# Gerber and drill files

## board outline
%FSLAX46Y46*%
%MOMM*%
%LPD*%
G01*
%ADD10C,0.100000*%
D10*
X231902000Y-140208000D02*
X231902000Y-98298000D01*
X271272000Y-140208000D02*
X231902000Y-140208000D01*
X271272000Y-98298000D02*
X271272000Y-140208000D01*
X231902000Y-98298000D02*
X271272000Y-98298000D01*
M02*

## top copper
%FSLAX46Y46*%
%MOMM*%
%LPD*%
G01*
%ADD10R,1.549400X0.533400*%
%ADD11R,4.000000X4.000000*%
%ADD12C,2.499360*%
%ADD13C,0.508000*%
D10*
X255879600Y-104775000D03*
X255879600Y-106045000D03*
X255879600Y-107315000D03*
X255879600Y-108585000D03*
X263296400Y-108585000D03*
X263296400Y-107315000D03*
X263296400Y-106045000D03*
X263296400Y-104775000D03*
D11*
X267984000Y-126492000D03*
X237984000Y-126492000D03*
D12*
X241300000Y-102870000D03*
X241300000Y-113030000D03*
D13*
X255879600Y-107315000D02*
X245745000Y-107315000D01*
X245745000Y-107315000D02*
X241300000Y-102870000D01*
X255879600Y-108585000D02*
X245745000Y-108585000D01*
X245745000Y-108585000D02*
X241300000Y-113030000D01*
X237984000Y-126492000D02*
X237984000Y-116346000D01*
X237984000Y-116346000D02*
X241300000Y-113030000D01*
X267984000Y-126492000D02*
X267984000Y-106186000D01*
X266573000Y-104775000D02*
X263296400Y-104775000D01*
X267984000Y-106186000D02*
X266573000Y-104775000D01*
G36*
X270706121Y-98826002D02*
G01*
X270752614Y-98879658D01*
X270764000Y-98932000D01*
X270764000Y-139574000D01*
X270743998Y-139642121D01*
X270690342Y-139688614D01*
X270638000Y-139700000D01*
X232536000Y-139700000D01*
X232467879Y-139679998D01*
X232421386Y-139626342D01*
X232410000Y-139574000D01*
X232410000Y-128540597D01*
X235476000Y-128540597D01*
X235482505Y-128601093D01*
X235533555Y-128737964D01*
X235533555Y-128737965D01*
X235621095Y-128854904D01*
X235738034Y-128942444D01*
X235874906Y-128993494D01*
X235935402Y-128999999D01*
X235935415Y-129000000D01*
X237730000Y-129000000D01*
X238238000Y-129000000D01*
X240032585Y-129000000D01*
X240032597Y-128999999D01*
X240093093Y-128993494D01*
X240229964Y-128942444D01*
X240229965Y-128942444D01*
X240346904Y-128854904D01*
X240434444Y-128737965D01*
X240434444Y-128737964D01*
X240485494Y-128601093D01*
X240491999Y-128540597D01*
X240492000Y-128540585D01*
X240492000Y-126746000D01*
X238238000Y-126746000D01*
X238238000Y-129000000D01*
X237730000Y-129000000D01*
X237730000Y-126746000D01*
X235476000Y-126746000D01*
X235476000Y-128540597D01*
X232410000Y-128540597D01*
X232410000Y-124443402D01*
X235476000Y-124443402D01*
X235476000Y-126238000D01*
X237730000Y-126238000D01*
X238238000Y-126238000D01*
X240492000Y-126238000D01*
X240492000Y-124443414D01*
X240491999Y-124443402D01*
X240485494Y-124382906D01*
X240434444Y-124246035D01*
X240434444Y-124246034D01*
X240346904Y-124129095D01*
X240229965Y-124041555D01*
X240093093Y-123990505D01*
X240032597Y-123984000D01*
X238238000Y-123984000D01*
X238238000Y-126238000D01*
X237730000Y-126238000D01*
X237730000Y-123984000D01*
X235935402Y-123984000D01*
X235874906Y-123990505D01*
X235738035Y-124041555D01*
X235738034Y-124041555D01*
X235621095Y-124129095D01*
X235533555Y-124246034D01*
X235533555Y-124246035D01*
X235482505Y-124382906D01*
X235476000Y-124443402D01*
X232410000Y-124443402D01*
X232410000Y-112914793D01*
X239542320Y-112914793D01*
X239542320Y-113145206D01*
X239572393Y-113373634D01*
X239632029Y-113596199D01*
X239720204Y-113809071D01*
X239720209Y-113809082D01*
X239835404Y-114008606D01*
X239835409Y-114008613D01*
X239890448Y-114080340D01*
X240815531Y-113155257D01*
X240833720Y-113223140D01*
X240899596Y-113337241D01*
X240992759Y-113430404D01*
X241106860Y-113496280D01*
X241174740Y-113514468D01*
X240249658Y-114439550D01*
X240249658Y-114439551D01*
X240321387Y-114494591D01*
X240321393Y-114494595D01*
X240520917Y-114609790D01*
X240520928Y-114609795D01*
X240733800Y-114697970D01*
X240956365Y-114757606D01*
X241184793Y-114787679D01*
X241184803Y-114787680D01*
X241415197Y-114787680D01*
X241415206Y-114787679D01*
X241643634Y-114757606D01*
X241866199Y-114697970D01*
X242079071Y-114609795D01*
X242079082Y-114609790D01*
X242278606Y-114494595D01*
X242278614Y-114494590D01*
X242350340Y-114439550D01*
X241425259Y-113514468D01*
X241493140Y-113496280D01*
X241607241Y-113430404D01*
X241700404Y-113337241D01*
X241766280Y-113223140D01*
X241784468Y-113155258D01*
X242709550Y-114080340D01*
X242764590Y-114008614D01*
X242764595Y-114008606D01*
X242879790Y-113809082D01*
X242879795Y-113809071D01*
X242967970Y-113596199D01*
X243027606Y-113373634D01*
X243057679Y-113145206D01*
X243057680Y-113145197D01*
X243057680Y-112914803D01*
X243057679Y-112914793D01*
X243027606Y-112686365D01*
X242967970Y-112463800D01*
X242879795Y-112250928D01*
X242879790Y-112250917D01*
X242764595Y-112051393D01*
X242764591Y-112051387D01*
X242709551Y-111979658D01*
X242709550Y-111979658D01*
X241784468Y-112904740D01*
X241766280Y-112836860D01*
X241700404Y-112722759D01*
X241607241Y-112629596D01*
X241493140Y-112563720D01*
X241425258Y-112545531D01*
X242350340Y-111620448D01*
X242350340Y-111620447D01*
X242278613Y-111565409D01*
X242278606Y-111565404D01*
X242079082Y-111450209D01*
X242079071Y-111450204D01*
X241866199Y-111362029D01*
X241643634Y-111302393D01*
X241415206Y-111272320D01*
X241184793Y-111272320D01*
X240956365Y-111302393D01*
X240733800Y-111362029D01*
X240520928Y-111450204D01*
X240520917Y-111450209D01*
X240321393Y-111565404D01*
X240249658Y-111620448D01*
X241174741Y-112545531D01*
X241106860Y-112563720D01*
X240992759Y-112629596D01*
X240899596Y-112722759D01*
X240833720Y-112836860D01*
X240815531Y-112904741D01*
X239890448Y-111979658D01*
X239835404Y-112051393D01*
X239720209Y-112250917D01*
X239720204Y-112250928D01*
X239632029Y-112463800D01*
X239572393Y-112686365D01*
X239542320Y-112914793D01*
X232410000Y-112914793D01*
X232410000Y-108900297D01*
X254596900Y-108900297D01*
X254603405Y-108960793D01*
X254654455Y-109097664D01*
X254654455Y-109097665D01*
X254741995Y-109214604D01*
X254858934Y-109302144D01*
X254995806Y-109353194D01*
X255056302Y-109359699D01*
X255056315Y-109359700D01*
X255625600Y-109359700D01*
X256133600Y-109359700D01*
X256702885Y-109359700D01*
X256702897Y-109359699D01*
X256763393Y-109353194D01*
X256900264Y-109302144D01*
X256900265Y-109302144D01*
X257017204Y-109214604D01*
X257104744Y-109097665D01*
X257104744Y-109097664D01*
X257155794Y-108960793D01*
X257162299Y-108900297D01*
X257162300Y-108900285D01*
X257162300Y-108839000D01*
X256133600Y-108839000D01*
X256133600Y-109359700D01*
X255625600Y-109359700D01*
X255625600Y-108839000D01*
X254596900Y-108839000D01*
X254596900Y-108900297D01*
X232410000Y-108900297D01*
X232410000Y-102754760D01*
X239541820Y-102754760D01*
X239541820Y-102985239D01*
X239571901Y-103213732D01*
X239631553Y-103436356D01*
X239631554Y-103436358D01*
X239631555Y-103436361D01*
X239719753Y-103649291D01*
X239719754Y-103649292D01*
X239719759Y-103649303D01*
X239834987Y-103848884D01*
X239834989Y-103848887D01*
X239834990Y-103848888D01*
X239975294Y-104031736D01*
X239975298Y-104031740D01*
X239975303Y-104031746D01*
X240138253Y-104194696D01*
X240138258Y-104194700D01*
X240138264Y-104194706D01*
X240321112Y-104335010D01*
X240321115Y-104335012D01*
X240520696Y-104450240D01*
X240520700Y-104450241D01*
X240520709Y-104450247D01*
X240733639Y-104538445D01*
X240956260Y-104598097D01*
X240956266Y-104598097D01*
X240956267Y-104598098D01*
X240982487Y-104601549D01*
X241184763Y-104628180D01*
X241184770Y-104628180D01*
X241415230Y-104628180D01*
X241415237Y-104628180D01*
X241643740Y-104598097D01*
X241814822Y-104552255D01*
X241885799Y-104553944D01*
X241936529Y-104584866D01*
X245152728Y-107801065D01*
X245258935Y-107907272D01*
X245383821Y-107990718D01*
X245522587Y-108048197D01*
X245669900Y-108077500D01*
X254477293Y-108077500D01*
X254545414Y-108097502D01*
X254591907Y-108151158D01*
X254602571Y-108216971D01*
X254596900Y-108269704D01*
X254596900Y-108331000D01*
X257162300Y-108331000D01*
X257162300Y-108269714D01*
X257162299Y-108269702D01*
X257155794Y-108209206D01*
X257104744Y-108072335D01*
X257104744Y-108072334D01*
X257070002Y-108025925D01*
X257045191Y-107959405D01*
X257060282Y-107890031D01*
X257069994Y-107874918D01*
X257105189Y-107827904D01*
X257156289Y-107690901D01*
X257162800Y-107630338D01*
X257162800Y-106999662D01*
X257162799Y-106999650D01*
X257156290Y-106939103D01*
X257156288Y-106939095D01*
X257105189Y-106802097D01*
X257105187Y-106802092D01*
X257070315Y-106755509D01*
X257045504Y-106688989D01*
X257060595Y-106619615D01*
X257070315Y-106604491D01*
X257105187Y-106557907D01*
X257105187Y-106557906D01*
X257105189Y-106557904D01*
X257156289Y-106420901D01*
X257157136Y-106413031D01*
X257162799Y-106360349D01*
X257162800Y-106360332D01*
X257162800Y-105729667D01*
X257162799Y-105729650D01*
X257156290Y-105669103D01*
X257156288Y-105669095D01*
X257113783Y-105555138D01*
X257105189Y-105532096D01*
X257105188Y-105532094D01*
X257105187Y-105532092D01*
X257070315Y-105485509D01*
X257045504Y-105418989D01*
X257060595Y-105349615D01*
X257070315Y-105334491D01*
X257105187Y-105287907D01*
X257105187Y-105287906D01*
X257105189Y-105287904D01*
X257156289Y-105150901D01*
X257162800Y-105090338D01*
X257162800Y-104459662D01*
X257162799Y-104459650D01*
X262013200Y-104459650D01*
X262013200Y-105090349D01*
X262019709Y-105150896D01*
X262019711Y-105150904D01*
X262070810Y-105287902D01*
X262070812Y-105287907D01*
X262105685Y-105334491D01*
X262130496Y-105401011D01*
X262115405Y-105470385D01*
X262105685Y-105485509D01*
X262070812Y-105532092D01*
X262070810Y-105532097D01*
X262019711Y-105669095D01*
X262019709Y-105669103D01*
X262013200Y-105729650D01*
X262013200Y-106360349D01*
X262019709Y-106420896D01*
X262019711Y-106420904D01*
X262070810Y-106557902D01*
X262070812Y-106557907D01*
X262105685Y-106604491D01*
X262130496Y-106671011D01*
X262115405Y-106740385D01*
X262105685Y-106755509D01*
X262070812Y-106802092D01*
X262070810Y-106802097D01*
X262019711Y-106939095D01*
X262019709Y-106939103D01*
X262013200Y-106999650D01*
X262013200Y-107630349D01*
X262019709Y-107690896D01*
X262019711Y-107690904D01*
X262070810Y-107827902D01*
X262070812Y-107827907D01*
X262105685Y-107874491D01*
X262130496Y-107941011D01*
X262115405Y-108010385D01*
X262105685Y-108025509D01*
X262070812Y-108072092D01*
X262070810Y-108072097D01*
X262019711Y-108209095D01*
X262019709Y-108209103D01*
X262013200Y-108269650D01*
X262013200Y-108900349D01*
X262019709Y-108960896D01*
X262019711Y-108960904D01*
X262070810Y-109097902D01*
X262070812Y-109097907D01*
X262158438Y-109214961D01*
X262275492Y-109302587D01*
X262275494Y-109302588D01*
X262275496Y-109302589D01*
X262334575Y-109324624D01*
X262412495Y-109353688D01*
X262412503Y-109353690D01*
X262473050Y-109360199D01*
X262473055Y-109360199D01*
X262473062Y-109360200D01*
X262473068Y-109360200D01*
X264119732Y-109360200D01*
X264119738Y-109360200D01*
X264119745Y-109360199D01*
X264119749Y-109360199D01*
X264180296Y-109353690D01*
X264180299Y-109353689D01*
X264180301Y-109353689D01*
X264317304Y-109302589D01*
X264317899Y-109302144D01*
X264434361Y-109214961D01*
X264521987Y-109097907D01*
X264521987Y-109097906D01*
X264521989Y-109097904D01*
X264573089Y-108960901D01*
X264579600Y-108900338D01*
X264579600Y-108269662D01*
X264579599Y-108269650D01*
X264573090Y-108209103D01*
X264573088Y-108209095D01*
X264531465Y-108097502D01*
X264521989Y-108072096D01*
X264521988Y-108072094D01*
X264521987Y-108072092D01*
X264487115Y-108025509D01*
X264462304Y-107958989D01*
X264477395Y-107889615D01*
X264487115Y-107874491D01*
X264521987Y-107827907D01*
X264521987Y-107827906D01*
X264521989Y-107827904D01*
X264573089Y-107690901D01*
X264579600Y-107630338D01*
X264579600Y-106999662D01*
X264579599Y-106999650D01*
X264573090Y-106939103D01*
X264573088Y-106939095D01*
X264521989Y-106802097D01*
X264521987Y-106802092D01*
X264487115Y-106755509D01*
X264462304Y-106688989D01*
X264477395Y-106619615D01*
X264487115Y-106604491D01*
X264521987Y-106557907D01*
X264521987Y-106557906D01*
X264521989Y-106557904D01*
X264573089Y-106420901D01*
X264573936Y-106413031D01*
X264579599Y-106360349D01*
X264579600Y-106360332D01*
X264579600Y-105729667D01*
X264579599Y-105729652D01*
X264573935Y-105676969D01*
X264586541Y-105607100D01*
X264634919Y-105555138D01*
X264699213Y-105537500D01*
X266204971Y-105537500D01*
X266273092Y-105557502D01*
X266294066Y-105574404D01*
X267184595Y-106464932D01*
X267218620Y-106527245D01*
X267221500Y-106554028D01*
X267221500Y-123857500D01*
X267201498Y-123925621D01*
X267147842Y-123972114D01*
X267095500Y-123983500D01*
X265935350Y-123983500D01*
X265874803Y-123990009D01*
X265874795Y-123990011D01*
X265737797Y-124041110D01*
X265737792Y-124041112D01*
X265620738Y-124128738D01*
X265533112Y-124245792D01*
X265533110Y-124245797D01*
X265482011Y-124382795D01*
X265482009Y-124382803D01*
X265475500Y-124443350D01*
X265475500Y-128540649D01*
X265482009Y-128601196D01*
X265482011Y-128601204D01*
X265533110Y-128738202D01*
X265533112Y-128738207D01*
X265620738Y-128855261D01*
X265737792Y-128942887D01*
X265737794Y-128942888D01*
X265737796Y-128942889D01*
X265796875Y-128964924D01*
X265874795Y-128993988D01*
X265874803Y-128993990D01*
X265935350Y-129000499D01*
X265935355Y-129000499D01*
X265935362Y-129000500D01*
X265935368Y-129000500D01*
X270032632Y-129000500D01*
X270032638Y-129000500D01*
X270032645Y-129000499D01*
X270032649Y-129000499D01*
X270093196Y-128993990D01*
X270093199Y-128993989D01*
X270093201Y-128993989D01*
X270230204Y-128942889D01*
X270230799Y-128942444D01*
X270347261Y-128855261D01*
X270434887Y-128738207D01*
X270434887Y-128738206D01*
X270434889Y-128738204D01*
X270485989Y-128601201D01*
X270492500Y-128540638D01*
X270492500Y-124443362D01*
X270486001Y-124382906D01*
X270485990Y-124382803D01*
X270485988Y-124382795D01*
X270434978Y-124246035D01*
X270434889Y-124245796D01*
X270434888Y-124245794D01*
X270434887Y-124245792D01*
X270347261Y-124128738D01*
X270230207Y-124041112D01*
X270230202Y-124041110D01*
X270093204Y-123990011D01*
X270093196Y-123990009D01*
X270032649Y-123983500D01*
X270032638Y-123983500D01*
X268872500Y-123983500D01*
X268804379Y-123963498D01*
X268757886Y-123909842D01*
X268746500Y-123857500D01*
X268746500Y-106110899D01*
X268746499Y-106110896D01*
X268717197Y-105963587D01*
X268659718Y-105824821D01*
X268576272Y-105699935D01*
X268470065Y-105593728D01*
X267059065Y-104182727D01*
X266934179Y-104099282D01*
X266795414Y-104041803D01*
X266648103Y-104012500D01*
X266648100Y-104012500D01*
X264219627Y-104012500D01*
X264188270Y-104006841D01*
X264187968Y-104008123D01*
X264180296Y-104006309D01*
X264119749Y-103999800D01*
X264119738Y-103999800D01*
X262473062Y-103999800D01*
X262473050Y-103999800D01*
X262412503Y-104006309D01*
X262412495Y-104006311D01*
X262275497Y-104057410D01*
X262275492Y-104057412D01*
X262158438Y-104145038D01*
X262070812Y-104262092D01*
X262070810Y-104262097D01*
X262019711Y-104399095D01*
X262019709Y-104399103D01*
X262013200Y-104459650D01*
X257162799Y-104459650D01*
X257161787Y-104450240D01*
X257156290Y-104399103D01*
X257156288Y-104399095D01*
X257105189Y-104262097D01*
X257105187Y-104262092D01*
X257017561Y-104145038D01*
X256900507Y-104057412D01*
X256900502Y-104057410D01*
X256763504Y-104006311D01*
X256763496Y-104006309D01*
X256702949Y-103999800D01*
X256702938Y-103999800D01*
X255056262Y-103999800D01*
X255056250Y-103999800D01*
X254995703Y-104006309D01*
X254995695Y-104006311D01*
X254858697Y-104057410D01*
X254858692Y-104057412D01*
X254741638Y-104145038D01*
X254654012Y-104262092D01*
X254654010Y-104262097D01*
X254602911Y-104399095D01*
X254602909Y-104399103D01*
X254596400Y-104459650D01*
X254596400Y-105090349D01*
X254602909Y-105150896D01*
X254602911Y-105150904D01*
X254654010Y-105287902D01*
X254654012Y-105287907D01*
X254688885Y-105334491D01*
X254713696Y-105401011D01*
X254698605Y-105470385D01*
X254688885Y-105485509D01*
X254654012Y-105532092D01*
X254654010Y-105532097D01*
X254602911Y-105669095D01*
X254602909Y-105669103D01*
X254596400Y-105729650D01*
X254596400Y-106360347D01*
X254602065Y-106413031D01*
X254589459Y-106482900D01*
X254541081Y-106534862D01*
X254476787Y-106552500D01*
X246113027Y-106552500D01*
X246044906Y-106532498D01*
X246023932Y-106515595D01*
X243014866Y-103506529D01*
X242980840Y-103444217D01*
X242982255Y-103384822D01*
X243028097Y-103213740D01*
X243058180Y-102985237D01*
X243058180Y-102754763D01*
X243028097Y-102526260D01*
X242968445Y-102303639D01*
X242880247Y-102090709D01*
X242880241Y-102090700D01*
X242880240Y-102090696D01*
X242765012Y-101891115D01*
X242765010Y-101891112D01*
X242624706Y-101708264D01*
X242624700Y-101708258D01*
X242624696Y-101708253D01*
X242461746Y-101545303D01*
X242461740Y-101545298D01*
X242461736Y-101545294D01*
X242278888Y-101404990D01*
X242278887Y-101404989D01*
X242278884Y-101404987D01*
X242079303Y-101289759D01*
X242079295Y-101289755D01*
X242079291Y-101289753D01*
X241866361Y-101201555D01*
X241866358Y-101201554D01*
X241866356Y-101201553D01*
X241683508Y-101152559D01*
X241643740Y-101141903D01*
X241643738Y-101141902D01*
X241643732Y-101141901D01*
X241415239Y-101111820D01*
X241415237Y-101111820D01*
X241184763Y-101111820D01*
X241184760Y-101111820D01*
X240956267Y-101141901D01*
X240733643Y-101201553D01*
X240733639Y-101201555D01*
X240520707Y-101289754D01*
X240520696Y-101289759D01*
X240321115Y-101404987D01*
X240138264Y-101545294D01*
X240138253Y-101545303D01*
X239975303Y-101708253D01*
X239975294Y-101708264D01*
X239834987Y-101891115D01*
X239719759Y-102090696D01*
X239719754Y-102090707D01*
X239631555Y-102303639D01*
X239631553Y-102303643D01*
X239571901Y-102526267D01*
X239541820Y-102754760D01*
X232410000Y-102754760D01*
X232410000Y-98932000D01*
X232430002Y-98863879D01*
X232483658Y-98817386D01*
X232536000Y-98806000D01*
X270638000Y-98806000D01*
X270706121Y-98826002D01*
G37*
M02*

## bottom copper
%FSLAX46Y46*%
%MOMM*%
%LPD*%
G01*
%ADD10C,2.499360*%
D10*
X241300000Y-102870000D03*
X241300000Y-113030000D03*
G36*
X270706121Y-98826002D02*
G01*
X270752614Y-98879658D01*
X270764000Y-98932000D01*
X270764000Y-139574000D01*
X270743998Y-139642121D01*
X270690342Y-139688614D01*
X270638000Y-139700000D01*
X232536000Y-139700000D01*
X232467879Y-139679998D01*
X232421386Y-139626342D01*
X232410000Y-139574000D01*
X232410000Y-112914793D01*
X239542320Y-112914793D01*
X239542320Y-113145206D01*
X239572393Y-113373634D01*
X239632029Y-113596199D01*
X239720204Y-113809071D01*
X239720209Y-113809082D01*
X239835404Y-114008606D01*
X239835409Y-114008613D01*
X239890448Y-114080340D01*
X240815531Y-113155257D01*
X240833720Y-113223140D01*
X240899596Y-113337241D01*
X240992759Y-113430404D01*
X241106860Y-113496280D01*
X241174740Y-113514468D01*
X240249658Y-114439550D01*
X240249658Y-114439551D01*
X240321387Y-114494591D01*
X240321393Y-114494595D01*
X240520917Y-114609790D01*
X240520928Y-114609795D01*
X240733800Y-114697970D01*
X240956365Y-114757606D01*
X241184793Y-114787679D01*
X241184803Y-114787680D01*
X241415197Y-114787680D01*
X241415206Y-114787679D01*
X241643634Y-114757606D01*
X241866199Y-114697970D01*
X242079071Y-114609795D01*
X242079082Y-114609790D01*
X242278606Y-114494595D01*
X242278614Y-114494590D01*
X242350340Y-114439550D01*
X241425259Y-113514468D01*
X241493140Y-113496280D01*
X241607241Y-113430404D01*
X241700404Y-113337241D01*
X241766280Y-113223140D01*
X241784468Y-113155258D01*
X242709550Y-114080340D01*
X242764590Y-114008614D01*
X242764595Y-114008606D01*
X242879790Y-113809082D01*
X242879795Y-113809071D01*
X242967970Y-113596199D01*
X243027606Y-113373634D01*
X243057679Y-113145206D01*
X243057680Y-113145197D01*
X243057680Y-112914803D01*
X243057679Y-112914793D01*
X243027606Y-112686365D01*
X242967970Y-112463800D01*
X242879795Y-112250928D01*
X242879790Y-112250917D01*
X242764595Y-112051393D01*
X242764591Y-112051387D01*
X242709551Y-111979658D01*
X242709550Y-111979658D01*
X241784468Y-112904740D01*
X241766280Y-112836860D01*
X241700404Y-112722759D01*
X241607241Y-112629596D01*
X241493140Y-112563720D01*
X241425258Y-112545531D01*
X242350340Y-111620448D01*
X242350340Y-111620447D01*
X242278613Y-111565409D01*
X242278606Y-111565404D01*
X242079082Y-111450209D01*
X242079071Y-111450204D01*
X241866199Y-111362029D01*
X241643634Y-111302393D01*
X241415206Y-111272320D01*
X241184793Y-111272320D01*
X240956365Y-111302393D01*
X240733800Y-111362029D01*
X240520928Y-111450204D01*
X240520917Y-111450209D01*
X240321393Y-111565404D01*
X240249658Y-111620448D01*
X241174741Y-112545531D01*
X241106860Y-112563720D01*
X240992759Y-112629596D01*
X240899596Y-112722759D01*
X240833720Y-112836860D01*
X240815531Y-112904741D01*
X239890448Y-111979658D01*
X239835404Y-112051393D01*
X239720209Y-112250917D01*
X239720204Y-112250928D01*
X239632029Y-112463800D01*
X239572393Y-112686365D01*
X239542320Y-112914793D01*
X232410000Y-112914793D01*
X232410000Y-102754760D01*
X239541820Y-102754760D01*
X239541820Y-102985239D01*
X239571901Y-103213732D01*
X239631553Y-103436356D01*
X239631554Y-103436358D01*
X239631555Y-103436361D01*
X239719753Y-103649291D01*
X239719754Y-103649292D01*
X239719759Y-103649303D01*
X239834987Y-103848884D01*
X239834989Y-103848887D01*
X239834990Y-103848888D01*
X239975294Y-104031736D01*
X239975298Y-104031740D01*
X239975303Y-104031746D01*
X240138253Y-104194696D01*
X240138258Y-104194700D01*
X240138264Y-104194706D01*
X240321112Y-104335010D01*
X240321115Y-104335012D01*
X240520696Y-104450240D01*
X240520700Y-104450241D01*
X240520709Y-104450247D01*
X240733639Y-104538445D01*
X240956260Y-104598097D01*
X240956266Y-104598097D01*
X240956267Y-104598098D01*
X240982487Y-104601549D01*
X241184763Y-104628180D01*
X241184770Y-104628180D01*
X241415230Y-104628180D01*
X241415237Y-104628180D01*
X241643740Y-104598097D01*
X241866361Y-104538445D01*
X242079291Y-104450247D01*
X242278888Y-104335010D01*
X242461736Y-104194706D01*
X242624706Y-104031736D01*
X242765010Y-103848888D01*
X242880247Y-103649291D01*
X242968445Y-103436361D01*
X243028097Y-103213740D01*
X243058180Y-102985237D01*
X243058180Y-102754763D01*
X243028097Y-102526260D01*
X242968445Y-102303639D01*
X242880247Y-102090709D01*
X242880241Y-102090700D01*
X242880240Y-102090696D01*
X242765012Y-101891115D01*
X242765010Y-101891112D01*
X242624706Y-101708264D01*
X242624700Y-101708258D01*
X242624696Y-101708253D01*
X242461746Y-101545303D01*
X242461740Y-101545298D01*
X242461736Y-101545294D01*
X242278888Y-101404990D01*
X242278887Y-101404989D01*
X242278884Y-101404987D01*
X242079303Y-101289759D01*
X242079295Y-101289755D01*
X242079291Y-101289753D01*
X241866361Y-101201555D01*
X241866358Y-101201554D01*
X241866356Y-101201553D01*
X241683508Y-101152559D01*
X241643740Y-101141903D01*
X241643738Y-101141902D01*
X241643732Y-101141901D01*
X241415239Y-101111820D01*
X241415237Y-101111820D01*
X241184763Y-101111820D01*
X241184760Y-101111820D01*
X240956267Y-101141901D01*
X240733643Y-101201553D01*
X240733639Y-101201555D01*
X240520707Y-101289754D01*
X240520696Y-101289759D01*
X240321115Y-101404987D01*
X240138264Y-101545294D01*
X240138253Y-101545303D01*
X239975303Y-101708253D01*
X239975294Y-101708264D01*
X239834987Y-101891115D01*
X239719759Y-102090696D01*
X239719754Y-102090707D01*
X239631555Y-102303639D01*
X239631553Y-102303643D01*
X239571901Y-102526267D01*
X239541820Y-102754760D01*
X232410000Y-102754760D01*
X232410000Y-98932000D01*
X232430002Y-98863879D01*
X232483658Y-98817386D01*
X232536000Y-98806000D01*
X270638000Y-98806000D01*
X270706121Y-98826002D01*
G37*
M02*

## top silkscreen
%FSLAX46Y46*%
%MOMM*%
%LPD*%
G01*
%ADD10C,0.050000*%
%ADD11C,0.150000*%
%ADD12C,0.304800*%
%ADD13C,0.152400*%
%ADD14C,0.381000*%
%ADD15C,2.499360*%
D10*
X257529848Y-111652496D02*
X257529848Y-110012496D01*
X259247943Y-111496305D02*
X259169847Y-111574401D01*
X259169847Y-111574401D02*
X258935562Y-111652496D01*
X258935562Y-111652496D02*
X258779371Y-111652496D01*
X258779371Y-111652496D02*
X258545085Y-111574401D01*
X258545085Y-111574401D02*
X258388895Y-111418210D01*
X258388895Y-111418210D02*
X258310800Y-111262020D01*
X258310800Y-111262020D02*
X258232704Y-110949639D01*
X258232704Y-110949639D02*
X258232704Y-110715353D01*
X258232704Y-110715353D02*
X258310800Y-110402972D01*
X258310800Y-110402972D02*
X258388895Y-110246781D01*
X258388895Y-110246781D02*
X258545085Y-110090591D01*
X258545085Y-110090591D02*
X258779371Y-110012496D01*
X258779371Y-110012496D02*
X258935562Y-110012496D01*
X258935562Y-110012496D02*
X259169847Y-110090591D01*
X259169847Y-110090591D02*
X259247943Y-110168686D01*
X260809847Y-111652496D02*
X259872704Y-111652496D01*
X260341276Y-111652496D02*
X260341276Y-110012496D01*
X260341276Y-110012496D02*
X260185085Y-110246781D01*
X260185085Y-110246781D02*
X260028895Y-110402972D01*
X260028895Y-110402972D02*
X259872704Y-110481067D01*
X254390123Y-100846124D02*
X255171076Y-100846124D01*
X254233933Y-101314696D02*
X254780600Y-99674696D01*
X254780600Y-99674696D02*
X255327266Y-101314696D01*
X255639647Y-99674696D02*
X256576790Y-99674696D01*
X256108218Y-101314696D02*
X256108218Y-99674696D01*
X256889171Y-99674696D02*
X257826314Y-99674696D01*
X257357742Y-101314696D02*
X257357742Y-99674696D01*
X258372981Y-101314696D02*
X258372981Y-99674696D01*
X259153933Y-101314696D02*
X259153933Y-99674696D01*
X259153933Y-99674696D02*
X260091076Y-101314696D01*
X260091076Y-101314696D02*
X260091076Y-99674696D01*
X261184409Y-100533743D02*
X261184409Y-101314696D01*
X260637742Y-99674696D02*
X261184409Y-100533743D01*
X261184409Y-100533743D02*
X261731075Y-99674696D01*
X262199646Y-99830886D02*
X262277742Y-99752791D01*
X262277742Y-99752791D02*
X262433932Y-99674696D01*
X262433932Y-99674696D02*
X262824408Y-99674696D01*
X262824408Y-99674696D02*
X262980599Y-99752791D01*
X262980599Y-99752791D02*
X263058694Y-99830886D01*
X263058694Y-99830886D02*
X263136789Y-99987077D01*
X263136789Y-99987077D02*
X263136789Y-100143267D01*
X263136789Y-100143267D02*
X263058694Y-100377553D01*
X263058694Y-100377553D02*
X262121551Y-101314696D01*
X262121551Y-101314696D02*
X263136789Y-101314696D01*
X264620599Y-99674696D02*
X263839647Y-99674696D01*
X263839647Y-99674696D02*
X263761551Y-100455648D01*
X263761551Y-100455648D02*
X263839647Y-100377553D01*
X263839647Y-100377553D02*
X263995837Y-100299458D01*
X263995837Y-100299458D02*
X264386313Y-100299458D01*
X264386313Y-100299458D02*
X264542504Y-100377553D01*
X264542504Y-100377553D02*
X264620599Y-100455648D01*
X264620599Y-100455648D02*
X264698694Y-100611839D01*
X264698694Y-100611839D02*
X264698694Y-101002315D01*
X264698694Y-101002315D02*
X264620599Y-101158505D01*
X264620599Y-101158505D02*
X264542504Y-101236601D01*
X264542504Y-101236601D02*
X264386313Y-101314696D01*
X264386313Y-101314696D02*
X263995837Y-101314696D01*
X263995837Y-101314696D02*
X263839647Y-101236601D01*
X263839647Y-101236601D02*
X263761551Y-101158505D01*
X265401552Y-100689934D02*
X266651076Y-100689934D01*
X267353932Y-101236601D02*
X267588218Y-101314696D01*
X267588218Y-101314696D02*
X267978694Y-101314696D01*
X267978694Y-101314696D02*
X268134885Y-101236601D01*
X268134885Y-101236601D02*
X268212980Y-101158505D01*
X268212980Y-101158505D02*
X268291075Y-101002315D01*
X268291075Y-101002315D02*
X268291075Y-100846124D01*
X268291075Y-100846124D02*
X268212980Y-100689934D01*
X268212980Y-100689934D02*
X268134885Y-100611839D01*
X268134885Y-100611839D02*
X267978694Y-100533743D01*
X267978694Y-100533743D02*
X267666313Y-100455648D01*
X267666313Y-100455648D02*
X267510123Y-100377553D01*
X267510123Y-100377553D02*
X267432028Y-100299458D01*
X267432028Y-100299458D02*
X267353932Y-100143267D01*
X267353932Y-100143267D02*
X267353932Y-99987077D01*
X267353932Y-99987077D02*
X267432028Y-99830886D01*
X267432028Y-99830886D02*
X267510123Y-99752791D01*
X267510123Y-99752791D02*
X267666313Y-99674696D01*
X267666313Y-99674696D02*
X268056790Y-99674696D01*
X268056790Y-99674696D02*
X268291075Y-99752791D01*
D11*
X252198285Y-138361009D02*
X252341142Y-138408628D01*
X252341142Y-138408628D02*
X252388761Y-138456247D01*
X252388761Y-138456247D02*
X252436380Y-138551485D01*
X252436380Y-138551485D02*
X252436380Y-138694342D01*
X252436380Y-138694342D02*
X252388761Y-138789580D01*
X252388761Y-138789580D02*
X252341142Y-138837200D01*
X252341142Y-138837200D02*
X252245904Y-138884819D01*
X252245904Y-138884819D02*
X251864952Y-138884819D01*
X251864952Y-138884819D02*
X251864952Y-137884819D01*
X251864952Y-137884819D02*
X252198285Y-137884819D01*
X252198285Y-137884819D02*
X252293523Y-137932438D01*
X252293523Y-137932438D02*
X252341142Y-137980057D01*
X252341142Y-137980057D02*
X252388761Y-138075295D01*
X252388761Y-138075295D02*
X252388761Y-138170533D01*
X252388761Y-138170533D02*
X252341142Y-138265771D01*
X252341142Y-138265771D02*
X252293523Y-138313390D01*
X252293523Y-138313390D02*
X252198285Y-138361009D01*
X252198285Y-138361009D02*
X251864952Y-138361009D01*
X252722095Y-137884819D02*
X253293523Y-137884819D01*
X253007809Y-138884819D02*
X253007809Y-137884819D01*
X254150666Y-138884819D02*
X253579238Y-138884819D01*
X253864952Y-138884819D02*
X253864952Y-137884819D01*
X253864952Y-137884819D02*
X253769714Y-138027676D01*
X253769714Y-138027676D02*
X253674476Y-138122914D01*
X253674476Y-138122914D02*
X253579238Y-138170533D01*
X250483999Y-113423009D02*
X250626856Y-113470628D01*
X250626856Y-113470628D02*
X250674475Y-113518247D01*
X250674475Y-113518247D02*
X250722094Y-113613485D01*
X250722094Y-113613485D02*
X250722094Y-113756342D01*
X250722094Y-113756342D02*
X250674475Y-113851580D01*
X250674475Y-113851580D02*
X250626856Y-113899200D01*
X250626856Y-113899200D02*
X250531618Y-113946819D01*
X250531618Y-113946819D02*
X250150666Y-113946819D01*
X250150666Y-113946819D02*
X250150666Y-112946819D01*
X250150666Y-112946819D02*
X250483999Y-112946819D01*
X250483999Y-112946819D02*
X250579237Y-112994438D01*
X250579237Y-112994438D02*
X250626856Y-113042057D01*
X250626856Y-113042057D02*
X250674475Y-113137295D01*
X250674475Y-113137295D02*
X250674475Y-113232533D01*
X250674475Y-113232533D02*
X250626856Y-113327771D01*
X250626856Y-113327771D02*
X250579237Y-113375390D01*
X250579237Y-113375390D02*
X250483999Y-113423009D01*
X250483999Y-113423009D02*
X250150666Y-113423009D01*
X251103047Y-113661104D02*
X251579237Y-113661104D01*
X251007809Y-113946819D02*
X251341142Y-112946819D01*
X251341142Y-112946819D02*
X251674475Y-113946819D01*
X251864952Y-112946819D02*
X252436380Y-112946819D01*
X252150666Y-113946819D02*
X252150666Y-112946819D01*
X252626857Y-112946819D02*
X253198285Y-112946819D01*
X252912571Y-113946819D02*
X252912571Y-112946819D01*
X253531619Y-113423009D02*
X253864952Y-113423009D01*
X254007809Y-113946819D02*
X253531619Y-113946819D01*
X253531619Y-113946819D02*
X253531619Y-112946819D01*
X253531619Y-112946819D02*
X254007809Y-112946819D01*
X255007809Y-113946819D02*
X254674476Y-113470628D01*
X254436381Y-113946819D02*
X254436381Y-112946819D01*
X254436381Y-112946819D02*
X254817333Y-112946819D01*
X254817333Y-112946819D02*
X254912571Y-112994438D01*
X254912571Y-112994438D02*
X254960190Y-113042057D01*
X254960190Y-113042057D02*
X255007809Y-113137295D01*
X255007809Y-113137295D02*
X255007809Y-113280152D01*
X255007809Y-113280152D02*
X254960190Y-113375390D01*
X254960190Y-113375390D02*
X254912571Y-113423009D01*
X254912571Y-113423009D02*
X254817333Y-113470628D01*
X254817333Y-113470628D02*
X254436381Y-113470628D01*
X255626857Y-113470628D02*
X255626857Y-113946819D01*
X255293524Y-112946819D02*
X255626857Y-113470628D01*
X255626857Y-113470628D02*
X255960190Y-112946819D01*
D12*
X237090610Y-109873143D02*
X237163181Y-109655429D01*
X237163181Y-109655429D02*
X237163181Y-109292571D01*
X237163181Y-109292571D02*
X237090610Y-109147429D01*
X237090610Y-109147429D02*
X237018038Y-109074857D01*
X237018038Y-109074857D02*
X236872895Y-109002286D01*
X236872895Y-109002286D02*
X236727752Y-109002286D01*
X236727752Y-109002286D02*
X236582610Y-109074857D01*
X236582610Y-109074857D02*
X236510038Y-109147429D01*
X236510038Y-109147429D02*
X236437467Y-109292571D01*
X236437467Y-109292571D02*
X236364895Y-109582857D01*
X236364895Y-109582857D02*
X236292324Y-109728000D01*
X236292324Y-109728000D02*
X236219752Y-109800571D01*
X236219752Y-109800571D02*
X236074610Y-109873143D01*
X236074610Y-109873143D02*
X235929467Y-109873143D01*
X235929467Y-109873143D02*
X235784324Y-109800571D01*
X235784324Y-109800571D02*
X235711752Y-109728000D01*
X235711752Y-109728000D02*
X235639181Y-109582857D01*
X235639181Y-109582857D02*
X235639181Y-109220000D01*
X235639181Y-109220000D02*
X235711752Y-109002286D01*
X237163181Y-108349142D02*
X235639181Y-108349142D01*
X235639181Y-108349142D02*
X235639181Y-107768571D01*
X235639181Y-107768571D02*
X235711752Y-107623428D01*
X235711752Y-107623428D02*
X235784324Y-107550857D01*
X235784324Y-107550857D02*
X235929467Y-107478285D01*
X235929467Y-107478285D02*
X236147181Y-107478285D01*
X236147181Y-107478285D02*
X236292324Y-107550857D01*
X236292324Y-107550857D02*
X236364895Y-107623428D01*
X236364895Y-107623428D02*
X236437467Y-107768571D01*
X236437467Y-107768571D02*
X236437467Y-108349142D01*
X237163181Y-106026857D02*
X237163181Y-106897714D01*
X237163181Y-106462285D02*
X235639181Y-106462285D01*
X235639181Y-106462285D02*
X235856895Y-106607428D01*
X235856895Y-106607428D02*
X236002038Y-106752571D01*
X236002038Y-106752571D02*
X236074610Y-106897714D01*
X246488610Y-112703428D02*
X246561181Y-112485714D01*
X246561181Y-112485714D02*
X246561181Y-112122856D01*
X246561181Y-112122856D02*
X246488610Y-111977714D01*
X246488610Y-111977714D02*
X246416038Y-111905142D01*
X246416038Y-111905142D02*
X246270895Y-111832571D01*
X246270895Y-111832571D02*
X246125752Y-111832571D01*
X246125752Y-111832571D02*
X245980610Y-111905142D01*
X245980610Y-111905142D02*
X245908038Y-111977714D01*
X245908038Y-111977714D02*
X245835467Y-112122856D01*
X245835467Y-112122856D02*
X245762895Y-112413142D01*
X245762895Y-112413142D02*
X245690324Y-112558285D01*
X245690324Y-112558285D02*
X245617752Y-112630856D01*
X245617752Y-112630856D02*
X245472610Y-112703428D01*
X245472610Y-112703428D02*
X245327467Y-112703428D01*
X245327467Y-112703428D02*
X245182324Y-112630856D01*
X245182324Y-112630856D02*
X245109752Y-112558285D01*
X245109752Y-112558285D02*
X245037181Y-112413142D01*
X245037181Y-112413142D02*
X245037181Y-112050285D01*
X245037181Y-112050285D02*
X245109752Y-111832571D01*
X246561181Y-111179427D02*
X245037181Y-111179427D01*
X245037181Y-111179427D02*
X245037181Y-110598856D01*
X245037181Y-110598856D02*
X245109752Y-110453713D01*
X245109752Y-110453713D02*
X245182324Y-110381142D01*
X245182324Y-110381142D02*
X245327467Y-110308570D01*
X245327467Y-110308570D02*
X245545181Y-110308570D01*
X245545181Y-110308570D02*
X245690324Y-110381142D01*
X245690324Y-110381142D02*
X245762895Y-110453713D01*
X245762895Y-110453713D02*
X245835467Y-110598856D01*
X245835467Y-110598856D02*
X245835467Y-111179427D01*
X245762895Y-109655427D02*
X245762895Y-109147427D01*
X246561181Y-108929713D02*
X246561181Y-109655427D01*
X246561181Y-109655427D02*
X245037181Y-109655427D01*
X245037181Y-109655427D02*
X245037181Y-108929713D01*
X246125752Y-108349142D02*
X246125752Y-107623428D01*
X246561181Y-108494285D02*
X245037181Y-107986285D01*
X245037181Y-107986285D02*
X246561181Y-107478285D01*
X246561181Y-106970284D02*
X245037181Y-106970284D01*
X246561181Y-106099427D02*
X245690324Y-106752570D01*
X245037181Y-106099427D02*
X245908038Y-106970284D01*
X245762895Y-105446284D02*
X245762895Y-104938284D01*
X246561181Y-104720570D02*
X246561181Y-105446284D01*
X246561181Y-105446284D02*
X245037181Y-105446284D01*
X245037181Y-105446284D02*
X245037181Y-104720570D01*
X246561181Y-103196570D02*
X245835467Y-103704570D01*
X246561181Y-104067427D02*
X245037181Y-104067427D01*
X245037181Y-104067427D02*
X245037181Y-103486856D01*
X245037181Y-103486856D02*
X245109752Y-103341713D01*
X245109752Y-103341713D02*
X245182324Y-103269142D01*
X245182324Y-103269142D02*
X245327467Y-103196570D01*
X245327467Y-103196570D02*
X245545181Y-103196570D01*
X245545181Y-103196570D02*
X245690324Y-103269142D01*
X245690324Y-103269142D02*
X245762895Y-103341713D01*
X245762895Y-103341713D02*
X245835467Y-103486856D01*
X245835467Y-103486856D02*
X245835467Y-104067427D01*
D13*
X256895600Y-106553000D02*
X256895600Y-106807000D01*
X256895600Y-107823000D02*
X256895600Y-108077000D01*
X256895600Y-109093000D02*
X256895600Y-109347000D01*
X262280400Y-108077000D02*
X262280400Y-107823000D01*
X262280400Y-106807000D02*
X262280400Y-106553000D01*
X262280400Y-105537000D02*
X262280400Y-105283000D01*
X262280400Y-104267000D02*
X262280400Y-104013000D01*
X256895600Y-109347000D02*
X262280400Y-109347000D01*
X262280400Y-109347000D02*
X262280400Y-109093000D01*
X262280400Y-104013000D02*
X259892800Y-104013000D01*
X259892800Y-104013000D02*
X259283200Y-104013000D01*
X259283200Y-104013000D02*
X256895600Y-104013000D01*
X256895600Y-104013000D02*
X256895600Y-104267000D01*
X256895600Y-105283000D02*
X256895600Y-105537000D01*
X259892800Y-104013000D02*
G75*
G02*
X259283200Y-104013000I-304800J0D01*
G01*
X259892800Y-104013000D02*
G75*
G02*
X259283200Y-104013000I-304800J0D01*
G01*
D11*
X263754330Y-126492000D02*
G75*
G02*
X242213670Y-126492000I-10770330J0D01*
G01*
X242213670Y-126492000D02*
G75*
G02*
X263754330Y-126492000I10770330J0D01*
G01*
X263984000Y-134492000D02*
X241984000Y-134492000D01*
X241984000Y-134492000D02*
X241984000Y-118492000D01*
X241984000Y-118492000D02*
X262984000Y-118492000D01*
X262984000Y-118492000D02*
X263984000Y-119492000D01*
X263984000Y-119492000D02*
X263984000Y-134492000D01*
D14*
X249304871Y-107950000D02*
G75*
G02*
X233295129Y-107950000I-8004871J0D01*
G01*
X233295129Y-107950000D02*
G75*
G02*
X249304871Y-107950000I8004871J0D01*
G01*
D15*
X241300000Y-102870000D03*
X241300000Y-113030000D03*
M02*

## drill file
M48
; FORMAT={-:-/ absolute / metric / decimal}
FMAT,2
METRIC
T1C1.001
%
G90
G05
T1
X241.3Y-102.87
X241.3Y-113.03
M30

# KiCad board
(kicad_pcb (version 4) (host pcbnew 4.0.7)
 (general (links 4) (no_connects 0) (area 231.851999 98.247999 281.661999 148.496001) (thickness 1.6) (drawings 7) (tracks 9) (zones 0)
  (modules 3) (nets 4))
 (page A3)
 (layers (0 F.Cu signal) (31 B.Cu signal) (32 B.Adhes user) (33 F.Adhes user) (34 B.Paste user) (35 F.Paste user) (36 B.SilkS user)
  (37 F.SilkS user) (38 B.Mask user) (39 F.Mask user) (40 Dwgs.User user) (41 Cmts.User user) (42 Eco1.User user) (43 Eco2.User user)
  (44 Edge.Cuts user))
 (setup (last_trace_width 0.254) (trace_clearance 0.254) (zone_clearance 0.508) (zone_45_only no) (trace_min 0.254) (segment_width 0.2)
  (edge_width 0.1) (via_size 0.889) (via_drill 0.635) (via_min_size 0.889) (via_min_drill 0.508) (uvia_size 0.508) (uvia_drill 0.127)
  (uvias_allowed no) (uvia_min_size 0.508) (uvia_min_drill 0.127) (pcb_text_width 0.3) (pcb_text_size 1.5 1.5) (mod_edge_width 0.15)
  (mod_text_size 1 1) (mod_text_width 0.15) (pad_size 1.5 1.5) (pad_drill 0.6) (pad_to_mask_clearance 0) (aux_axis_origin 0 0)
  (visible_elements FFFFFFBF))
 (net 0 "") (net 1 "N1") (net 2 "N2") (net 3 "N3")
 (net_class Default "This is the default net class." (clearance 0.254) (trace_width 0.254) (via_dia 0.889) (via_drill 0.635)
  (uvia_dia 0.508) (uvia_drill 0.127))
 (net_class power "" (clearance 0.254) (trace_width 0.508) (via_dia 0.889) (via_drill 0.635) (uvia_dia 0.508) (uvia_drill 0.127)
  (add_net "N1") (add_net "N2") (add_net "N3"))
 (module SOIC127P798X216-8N (layer F.Cu) (at 259.588 106.68) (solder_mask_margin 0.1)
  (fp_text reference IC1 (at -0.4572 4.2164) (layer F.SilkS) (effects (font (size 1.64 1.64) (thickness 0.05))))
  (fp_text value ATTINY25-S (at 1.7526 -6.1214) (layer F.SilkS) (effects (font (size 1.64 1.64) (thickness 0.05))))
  (fp_line (start -2.6924 -0.127) (end -2.6924 0.127) (layer F.SilkS) (width 0.1524))
  (fp_line (start -2.6924 1.143) (end -2.6924 1.397) (layer F.SilkS) (width 0.1524))
  (fp_line (start -2.6924 2.413) (end -2.6924 2.667) (layer F.SilkS) (width 0.1524))
  (fp_line (start 2.6924 1.397) (end 2.6924 1.143) (layer F.SilkS) (width 0.1524))
  (fp_line (start 2.6924 0.127) (end 2.6924 -0.127) (layer F.SilkS) (width 0.1524))
  (fp_line (start 2.6924 -1.143) (end 2.6924 -1.397) (layer F.SilkS) (width 0.1524))
  (fp_line (start 2.6924 -2.413) (end 2.6924 -2.667) (layer F.SilkS) (width 0.1524))
  (fp_line (start -2.6924 2.667) (end 2.6924 2.667) (layer F.SilkS) (width 0.1524))
  (fp_line (start 2.6924 2.667) (end 2.6924 2.413) (layer F.SilkS) (width 0.1524))
  (fp_line (start 2.6924 -2.667) (end 0.3048 -2.667) (layer F.SilkS) (width 0.1524))
  (fp_line (start 0.3048 -2.667) (end -0.3048 -2.667) (layer F.SilkS) (width 0.1524))
  (fp_line (start -0.3048 -2.667) (end -2.6924 -2.667) (layer F.SilkS) (width 0.1524))
  (fp_line (start -2.6924 -2.667) (end -2.6924 -2.413) (layer F.SilkS) (width 0.1524))
  (fp_line (start -2.6924 -1.397) (end -2.6924 -1.143) (layer F.SilkS) (width 0.1524))
  (fp_arc (start 0 -2.667) (end -0.3048 -2.667) (angle -180) (layer F.SilkS) (width 0.1524))
  (fp_arc (start 0 -2.667) (end -0.3048 -2.667) (angle -180) (layer F.SilkS) (width 0.1524))
  (pad 1 smd rect (at -3.7084 -1.905) (size 1.5494 0.5334) (layers F.Cu F.Paste F.Mask) (solder_mask_margin 0.2))
  (pad 2 smd rect (at -3.7084 -0.635) (size 1.5494 0.5334) (layers F.Cu F.Paste F.Mask) (solder_mask_margin 0.2))
  (pad 3 smd rect (at -3.7084 0.635) (size 1.5494 0.5334) (layers F.Cu F.Paste F.Mask) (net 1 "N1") (solder_mask_margin 0.2))
  (pad 4 smd rect (at -3.7084 1.905) (size 1.5494 0.5334) (layers F.Cu F.Paste F.Mask) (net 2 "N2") (solder_mask_margin 0.2))
  (pad 5 smd rect (at 3.7084 1.905) (size 1.5494 0.5334) (layers F.Cu F.Paste F.Mask) (solder_mask_margin 0.2))
  (pad 6 smd rect (at 3.7084 0.635) (size 1.5494 0.5334) (layers F.Cu F.Paste F.Mask) (solder_mask_margin 0.2))
  (pad 7 smd rect (at 3.7084 -0.635) (size 1.5494 0.5334) (layers F.Cu F.Paste F.Mask) (solder_mask_margin 0.2))
  (pad 8 smd rect (at 3.7084 -1.905) (size 1.5494 0.5334) (layers F.Cu F.Paste F.Mask) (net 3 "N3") (solder_mask_margin 0.2)))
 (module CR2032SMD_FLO (layer F.Cu) (at 252.984 126.492 180)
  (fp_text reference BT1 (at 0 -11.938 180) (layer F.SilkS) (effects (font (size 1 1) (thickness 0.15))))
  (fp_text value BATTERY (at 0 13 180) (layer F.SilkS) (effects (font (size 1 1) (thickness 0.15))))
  (fp_circle (center 0 0) (end -4 -10) (layer F.SilkS) (width 0.15))
  (fp_line (start -11 -8) (end 11 -8) (layer F.SilkS) (width 0.15))
  (fp_line (start 11 -8) (end 11 8) (layer F.SilkS) (width 0.15))
  (fp_line (start 11 8) (end -10 8) (layer F.SilkS) (width 0.15))
  (fp_line (start -10 8) (end -11 7) (layer F.SilkS) (width 0.15))
  (fp_line (start -11 7) (end -11 -8) (layer F.SilkS) (width 0.15))
  (pad 1 smd rect (at -15 0 180) (size 4 4) (layers F.Cu F.Paste F.Mask) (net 3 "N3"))
  (pad 2 smd rect (at 15 0 180) (size 4 4) (layers F.Cu F.Paste F.Mask) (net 2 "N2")))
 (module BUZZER (layer F.Cu) (at 241.3 107.95 90)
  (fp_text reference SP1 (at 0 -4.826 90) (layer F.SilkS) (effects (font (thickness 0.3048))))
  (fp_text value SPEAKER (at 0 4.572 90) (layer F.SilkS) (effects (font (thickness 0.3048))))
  (fp_circle (center 0 0) (end 8.001 0.24892) (layer F.SilkS) (width 0.381))
  (pad 2 thru_hole circle (at 5.08 0 90) (size 2.49936 2.49936) (drill 1.00076) (layers *.Cu *.Mask F.SilkS) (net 1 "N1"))
  (pad 1 thru_hole circle (at -5.08 0 90) (size 2.49936 2.49936) (drill 1.00076) (layers *.Cu *.Mask F.SilkS) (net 2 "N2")))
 (gr_line (start 231.902 140.208) (end 231.902 98.298) (angle 90) (layer Edge.Cuts) (width 0.1))
 (gr_line (start 271.272 140.208) (end 231.902 140.208) (angle 90) (layer Edge.Cuts) (width 0.1))
 (gr_line (start 271.272 98.298) (end 271.272 140.208) (angle 90) (layer Edge.Cuts) (width 0.1))
 (gr_line (start 231.902 98.298) (end 271.272 98.298) (angle 90) (layer Edge.Cuts) (width 0.1))
 (segment (start 255.8796 107.315) (end 245.745 107.315) (width 0.508) (layer F.Cu) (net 1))
 (segment (start 245.745 107.315) (end 241.3 102.87) (width 0.508) (layer F.Cu) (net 1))
 (segment (start 255.8796 108.585) (end 245.745 108.585) (width 0.508) (layer F.Cu) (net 2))
 (segment (start 245.745 108.585) (end 241.3 113.03) (width 0.508) (layer F.Cu) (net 2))
 (segment (start 237.984 126.492) (end 237.984 116.346) (width 0.508) (layer F.Cu) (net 2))
 (segment (start 237.984 116.346) (end 241.3 113.03) (width 0.508) (layer F.Cu) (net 2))
 (segment (start 267.984 126.492) (end 267.984 106.186) (width 0.508) (layer F.Cu) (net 3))
 (segment (start 266.573 104.775) (end 263.2964 104.775) (width 0.508) (layer F.Cu) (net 3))
 (segment (start 267.984 106.186) (end 266.573 104.775) (width 0.508) (layer F.Cu) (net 3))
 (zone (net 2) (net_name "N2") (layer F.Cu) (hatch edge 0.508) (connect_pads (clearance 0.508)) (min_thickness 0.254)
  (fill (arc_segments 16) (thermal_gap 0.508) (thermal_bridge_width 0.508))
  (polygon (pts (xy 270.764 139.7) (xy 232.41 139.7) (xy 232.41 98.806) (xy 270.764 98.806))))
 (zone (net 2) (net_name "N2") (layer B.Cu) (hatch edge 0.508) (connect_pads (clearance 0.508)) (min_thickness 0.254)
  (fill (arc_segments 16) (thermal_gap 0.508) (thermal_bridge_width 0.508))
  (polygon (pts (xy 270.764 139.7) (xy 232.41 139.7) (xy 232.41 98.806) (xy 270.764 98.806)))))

